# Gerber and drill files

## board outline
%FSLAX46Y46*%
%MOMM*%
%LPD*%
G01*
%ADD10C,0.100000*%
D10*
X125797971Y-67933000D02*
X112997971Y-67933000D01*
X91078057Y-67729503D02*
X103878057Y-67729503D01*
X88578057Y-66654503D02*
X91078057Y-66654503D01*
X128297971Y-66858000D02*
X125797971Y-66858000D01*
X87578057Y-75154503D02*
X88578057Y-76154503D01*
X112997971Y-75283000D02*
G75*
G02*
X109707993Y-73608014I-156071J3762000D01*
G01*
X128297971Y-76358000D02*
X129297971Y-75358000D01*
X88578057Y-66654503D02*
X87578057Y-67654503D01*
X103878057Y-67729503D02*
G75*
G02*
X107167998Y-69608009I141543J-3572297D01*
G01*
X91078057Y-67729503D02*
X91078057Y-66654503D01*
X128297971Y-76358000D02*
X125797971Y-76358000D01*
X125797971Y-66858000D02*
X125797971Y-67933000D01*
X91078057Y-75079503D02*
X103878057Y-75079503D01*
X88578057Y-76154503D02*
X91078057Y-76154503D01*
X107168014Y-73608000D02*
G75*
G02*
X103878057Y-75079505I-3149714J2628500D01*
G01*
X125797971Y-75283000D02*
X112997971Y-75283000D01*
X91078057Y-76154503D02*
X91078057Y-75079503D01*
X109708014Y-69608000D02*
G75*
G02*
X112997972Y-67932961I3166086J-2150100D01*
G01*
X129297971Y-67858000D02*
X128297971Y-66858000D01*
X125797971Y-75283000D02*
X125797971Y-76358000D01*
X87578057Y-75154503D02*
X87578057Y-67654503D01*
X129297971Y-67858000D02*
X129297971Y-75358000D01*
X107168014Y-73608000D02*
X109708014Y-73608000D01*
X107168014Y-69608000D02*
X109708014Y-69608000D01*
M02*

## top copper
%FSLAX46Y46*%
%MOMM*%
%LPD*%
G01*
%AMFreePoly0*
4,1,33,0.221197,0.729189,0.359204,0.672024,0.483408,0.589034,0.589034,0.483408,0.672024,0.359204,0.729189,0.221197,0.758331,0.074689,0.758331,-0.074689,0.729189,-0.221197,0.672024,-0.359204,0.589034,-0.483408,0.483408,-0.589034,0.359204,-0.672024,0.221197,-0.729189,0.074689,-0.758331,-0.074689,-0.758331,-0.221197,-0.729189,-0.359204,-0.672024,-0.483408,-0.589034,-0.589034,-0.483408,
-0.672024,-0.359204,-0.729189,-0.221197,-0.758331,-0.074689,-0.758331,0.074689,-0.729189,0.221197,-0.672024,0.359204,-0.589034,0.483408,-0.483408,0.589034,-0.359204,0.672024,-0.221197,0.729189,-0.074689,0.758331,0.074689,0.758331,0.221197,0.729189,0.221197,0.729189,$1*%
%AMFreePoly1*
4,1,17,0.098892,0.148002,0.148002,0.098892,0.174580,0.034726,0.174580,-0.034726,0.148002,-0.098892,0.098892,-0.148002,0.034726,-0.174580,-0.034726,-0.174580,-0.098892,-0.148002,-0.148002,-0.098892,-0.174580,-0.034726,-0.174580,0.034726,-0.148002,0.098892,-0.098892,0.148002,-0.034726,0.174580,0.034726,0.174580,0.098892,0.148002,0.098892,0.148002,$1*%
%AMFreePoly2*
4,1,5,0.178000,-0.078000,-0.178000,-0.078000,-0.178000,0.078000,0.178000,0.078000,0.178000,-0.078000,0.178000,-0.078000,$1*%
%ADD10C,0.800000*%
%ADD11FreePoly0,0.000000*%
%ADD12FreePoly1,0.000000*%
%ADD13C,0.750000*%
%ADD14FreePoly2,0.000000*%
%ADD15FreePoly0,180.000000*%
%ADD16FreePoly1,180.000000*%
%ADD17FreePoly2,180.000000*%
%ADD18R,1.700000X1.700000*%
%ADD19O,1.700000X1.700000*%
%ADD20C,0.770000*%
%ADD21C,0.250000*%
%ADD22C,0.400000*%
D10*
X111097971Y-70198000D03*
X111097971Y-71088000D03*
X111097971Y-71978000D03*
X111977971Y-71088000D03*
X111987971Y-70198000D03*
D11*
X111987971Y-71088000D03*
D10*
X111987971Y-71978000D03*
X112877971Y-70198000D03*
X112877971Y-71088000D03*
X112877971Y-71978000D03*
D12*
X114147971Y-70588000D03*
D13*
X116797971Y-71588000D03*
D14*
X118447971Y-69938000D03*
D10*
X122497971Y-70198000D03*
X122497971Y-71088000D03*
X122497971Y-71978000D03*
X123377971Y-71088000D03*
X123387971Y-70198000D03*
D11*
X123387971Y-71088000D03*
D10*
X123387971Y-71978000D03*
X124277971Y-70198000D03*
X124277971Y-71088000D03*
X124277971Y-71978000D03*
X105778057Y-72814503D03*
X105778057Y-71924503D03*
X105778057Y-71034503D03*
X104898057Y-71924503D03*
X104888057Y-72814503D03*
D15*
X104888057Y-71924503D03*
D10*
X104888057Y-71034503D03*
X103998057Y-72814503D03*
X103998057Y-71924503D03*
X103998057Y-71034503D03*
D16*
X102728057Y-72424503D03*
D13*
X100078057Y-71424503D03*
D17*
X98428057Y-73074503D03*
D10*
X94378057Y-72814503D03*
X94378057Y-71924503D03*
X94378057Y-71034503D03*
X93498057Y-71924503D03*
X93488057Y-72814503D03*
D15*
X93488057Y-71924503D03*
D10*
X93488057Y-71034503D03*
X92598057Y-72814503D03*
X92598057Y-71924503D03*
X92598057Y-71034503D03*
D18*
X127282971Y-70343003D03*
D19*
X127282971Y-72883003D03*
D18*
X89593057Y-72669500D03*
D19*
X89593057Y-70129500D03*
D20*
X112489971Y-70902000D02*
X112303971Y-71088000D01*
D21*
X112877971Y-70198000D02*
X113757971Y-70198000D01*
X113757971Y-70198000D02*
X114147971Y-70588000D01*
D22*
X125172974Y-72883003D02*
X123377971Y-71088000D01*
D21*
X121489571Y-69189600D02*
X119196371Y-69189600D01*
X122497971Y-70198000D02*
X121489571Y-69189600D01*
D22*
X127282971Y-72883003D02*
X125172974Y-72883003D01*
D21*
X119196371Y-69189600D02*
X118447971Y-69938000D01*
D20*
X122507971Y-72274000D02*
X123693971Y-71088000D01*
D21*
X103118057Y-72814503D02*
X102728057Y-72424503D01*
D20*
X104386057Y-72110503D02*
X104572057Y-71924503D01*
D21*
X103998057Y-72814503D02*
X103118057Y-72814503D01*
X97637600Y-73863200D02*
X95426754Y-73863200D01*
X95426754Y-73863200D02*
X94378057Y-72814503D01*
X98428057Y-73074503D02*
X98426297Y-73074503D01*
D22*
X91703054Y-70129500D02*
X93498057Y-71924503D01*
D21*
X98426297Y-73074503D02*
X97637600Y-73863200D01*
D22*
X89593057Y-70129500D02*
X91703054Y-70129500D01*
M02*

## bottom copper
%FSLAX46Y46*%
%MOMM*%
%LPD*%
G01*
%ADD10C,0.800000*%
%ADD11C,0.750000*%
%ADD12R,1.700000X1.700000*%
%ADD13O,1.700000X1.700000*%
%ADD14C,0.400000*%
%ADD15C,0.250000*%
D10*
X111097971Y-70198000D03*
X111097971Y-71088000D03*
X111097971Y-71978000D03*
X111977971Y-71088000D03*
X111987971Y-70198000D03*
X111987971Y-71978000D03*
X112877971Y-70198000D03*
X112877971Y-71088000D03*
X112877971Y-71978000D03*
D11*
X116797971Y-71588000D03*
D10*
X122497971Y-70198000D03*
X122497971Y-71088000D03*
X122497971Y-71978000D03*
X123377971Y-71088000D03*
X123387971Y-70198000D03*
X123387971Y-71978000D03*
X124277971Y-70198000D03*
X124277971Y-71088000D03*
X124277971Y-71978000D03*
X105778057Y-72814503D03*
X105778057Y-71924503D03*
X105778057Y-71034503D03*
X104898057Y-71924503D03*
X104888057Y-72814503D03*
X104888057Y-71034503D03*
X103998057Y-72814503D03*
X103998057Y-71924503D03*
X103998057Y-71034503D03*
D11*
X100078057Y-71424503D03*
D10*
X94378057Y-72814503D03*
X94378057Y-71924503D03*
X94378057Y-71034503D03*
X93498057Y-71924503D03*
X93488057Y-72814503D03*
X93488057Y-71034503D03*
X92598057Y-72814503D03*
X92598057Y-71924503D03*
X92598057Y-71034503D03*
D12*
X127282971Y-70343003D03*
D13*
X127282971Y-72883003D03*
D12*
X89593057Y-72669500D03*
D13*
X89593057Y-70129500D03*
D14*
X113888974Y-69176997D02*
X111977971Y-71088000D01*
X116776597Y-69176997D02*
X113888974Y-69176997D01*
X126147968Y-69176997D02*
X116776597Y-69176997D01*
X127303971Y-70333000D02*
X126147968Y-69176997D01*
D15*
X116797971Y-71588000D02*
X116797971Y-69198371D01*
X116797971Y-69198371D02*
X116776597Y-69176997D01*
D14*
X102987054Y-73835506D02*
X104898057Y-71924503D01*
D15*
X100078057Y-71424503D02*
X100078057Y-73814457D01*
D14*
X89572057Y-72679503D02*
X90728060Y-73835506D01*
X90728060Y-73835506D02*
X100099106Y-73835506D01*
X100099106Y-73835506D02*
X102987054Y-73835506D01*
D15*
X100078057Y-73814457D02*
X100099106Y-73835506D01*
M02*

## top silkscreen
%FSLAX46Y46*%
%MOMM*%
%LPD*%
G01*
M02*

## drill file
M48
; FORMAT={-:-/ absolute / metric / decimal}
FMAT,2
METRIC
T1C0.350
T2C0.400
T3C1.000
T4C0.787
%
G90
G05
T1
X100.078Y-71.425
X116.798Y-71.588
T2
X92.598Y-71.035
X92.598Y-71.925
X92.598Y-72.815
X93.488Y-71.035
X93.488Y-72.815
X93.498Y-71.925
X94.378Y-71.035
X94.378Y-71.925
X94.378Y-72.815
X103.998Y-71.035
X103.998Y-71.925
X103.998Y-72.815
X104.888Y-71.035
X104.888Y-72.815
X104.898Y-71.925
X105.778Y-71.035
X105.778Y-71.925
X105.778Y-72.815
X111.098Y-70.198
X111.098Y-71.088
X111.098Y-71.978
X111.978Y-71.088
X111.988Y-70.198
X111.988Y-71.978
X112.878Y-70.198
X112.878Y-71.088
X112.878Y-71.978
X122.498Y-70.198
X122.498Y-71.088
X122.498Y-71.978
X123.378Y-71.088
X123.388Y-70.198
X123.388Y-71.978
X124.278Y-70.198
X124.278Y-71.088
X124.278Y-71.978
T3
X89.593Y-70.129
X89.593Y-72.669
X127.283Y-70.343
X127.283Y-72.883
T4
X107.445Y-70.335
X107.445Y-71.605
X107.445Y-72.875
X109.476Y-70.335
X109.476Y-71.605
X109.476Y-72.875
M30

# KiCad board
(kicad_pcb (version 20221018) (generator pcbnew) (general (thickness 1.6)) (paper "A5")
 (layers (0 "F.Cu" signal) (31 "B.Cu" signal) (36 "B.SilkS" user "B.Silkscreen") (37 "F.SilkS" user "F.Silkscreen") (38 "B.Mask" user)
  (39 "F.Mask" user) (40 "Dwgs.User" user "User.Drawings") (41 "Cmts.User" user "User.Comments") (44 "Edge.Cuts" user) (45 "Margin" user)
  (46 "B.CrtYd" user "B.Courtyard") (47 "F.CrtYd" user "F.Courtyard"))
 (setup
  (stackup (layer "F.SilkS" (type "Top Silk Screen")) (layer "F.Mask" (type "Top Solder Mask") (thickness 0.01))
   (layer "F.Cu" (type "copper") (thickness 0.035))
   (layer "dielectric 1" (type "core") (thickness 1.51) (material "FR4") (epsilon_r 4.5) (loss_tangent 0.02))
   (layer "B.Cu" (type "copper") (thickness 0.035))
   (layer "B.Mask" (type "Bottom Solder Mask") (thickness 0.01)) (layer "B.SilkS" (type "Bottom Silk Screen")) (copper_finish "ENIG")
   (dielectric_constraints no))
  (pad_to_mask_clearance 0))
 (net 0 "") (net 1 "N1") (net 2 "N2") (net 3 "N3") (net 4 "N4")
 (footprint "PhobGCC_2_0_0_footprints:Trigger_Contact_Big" (layer "F.Cu") (at 116.797971 71.588)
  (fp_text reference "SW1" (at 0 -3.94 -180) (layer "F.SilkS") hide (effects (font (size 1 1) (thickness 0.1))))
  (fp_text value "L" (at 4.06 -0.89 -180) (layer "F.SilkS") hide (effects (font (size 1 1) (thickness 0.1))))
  (pad "1" thru_hole circle (at -5.7 -1.39) (size 0.8 0.8) (drill 0.4) (layers "*.Cu" "*.Mask") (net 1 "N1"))
  (pad "1" thru_hole circle (at -5.7 -0.5) (size 0.8 0.8) (drill 0.4) (layers "*.Cu" "*.Mask") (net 1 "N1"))
  (pad "1" thru_hole circle (at -5.7 0.39) (size 0.8 0.8) (drill 0.4) (layers "*.Cu" "*.Mask") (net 1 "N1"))
  (pad "1" thru_hole circle (at -4.82 -0.5) (size 0.8 0.8) (drill 0.4) (layers "*.Cu" "*.Mask") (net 1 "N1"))
  (pad "1" thru_hole circle (at -4.81 -1.39) (size 0.8 0.8) (drill 0.4) (layers "*.Cu" "*.Mask") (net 1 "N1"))
  (pad "1" smd custom (at -4.81 -0.5) (size 1.524 1.524) (layers "F.Cu" "F.Paste" "F.Mask") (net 1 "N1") (thermal_bridge_angle 45)
   (options (clearance outline) (anchor circle)) (primitives))
  (pad "1" thru_hole circle (at -4.81 0.39) (size 0.8 0.8) (drill 0.4) (layers "*.Cu" "*.Mask") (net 1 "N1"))
  (pad "1" thru_hole circle (at -3.92 -1.39) (size 0.8 0.8) (drill 0.4) (layers "*.Cu" "*.Mask") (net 1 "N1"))
  (pad "1" thru_hole circle (at -3.92 -0.5) (size 0.8 0.8) (drill 0.4) (layers "*.Cu" "*.Mask") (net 1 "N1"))
  (pad "1" thru_hole circle (at -3.92 0.39) (size 0.8 0.8) (drill 0.4) (layers "*.Cu" "*.Mask") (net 1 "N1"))
  (pad "1" smd custom (at -2.65 -1) (size 0.356 0.356) (layers "F.Cu" "F.Paste" "F.Mask") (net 1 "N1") (thermal_bridge_angle 45)
   (options (clearance outline) (anchor circle)) (primitives))
  (pad "1" thru_hole circle (at 0 0) (size 0.75 0.75) (drill 0.35) (layers "*.Cu" "*.Mask") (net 1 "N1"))
  (pad "2" smd custom (at 1.65 -1.65) (size 0.356 0.156) (layers "F.Cu" "F.Paste" "F.Mask") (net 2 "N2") (thermal_bridge_angle 45)
   (options (clearance outline) (anchor rect)) (primitives))
  (pad "2" thru_hole circle (at 5.7 -1.39) (size 0.8 0.8) (drill 0.4) (layers "*.Cu" "*.Mask") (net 2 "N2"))
  (pad "2" thru_hole circle (at 5.7 -0.5) (size 0.8 0.8) (drill 0.4) (layers "*.Cu" "*.Mask") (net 2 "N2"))
  (pad "2" thru_hole circle (at 5.7 0.39) (size 0.8 0.8) (drill 0.4) (layers "*.Cu" "*.Mask") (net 2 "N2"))
  (pad "2" thru_hole circle (at 6.58 -0.5) (size 0.8 0.8) (drill 0.4) (layers "*.Cu" "*.Mask") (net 2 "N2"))
  (pad "2" thru_hole circle (at 6.59 -1.39) (size 0.8 0.8) (drill 0.4) (layers "*.Cu" "*.Mask") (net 2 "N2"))
  (pad "2" smd custom (at 6.59 -0.5) (size 1.524 1.524) (layers "F.Cu" "F.Paste" "F.Mask") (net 2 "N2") (thermal_bridge_angle 45)
   (options (clearance outline) (anchor circle)) (primitives))
  (pad "2" thru_hole circle (at 6.59 0.39) (size 0.8 0.8) (drill 0.4) (layers "*.Cu" "*.Mask") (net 2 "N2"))
  (pad "2" thru_hole circle (at 7.48 -1.39) (size 0.8 0.8) (drill 0.4) (layers "*.Cu" "*.Mask") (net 2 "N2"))
  (pad "2" thru_hole circle (at 7.48 -0.5) (size 0.8 0.8) (drill 0.4) (layers "*.Cu" "*.Mask") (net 2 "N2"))
  (pad "2" thru_hole circle (at 7.48 0.39) (size 0.8 0.8) (drill 0.4) (layers "*.Cu" "*.Mask") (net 2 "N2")))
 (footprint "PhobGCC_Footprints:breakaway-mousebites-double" (layer "F.Cu") (at 109.705907 71.375 90)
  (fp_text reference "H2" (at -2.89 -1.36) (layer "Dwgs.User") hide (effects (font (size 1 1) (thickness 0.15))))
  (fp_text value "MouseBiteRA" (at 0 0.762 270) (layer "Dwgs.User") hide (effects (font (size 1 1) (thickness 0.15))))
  (fp_line (start -2.233 -2.537893) (end -2.233 0.002107) (stroke (width 0.1) (type solid)) (layer "Edge.Cuts"))
  (fp_line (start 1.767 -2.537893) (end 1.767 0.002107) (stroke (width 0.1) (type solid)) (layer "Edge.Cuts"))
  (pad "" np_thru_hole circle (at -1.5 -2.26085 270) (size 0.7874 0.7874) (drill 0.7874) (layers "*.Cu" "*.Mask"))
  (pad "" np_thru_hole circle (at -1.5 -0.23 90) (size 0.7874 0.7874) (drill 0.7874) (layers "*.Cu" "*.Mask"))
  (pad "" np_thru_hole circle (at -0.23 -2.26085 270) (size 0.7874 0.7874) (drill 0.7874) (layers "*.Cu" "*.Mask"))
  (pad "" np_thru_hole circle (at -0.23 -0.23 90) (size 0.7874 0.7874) (drill 0.7874) (layers "*.Cu" "*.Mask"))
  (pad "" np_thru_hole circle (at 1.04 -2.26085 270) (size 0.7874 0.7874) (drill 0.7874) (layers "*.Cu" "*.Mask"))
  (pad "" np_thru_hole circle (at 1.04 -0.23 90) (size 0.7874 0.7874) (drill 0.7874) (layers "*.Cu" "*.Mask")))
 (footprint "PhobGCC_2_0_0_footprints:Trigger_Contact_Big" (layer "F.Cu") (at 100.078057 71.424503 180)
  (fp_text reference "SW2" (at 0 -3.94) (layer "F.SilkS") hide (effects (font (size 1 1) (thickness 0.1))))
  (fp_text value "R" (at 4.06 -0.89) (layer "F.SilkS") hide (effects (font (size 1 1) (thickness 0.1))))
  (pad "1" thru_hole circle (at -5.7 -1.39 180) (size 0.8 0.8) (drill 0.4) (layers "*.Cu" "*.Mask") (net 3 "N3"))
  (pad "1" thru_hole circle (at -5.7 -0.5 180) (size 0.8 0.8) (drill 0.4) (layers "*.Cu" "*.Mask") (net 3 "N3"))
  (pad "1" thru_hole circle (at -5.7 0.39 180) (size 0.8 0.8) (drill 0.4) (layers "*.Cu" "*.Mask") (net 3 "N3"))
  (pad "1" thru_hole circle (at -4.82 -0.5 180) (size 0.8 0.8) (drill 0.4) (layers "*.Cu" "*.Mask") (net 3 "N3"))
  (pad "1" thru_hole circle (at -4.81 -1.39 180) (size 0.8 0.8) (drill 0.4) (layers "*.Cu" "*.Mask") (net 3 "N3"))
  (pad "1" smd custom (at -4.81 -0.5 180) (size 1.524 1.524) (layers "F.Cu" "F.Paste" "F.Mask") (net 3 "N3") (thermal_bridge_angle 45)
   (options (clearance outline) (anchor circle)) (primitives))
  (pad "1" thru_hole circle (at -4.81 0.39 180) (size 0.8 0.8) (drill 0.4) (layers "*.Cu" "*.Mask") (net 3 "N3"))
  (pad "1" thru_hole circle (at -3.92 -1.39 180) (size 0.8 0.8) (drill 0.4) (layers "*.Cu" "*.Mask") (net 3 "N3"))
  (pad "1" thru_hole circle (at -3.92 -0.5 180) (size 0.8 0.8) (drill 0.4) (layers "*.Cu" "*.Mask") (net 3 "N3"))
  (pad "1" thru_hole circle (at -3.92 0.39 180) (size 0.8 0.8) (drill 0.4) (layers "*.Cu" "*.Mask") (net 3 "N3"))
  (pad "1" smd custom (at -2.65 -1 180) (size 0.356 0.356) (layers "F.Cu" "F.Paste" "F.Mask") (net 3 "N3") (thermal_bridge_angle 45)
   (options (clearance outline) (anchor circle)) (primitives))
  (pad "1" thru_hole circle (at 0 0 180) (size 0.75 0.75) (drill 0.35) (layers "*.Cu" "*.Mask") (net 3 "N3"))
  (pad "2" smd custom (at 1.65 -1.65 180) (size 0.356 0.156) (layers "F.Cu" "F.Paste" "F.Mask") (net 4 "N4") (thermal_bridge_angle 45)
   (options (clearance outline) (anchor rect)) (primitives))
  (pad "2" thru_hole circle (at 5.7 -1.39 180) (size 0.8 0.8) (drill 0.4) (layers "*.Cu" "*.Mask") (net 4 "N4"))
  (pad "2" thru_hole circle (at 5.7 -0.5 180) (size 0.8 0.8) (drill 0.4) (layers "*.Cu" "*.Mask") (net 4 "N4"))
  (pad "2" thru_hole circle (at 5.7 0.39 180) (size 0.8 0.8) (drill 0.4) (layers "*.Cu" "*.Mask") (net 4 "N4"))
  (pad "2" thru_hole circle (at 6.58 -0.5 180) (size 0.8 0.8) (drill 0.4) (layers "*.Cu" "*.Mask") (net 4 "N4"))
  (pad "2" thru_hole circle (at 6.59 -1.39 180) (size 0.8 0.8) (drill 0.4) (layers "*.Cu" "*.Mask") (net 4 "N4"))
  (pad "2" smd custom (at 6.59 -0.5 180) (size 1.524 1.524) (layers "F.Cu" "F.Paste" "F.Mask") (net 4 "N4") (thermal_bridge_angle 45)
   (options (clearance outline) (anchor circle)) (primitives))
  (pad "2" thru_hole circle (at 6.59 0.39 180) (size 0.8 0.8) (drill 0.4) (layers "*.Cu" "*.Mask") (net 4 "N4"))
  (pad "2" thru_hole circle (at 7.48 -1.39 180) (size 0.8 0.8) (drill 0.4) (layers "*.Cu" "*.Mask") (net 4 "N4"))
  (pad "2" thru_hole circle (at 7.48 -0.5 180) (size 0.8 0.8) (drill 0.4) (layers "*.Cu" "*.Mask") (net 4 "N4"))
  (pad "2" thru_hole circle (at 7.48 0.39 180) (size 0.8 0.8) (drill 0.4) (layers "*.Cu" "*.Mask") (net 4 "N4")))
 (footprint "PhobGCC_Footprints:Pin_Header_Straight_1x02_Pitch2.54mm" (layer "B.Cu") (at 127.282971 70.343003 180)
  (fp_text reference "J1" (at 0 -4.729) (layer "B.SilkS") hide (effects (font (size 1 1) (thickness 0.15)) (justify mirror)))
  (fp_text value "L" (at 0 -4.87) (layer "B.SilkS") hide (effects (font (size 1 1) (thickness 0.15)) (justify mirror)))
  (pad "1" thru_hole rect (at 0 0 180) (size 1.7 1.7) (drill 1) (layers "*.Cu" "*.Mask") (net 1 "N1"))
  (pad "2" thru_hole oval (at 0 -2.54 180) (size 1.7 1.7) (drill 1) (layers "*.Cu" "*.Mask") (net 2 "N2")))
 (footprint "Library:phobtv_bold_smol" (layer "B.Cu") (at 118.4 71.7)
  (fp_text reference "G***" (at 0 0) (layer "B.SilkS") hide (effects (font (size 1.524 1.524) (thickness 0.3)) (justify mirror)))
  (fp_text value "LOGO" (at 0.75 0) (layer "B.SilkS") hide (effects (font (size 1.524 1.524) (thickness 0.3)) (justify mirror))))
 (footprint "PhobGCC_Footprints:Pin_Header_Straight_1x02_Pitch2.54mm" (layer "B.Cu") (at 89.593057 72.6695)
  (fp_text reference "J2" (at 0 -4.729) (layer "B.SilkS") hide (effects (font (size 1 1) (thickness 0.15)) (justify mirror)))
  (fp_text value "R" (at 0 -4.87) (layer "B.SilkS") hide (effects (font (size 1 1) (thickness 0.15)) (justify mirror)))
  (pad "1" thru_hole rect (at 0 0) (size 1.7 1.7) (drill 1) (layers "*.Cu" "*.Mask") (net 3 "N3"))
  (pad "2" thru_hole oval (at 0 -2.54) (size 1.7 1.7) (drill 1) (layers "*.Cu" "*.Mask") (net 4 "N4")))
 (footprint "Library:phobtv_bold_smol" (layer "B.Cu") (at 98.5 71.3 180)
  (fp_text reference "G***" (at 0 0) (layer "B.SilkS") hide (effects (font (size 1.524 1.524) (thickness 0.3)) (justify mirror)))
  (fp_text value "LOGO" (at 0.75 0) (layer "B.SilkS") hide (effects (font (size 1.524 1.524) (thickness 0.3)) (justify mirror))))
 (gr_line (start 125.797971 67.933) (end 112.997971 67.933) (stroke (width 0.1) (type solid)) (layer "Edge.Cuts"))
 (gr_line (start 91.078057 67.729503) (end 103.878057 67.729503) (stroke (width 0.1) (type solid)) (layer "Edge.Cuts"))
 (gr_line (start 88.578057 66.654503) (end 91.078057 66.654503) (stroke (width 0.1) (type solid)) (layer "Edge.Cuts"))
 (gr_line (start 128.297971 66.858) (end 125.797971 66.858) (stroke (width 0.1) (type solid)) (layer "Edge.Cuts"))
 (gr_line (start 87.578057 75.154503) (end 88.578057 76.154503) (stroke (width 0.1) (type solid)) (layer "Edge.Cuts"))
 (gr_arc (start 112.997971 75.283) (mid 111.133614 74.876392) (end 109.708014 73.608) (stroke (width 0.1) (type solid)) (layer "Edge.Cuts"))
 (gr_line (start 128.297971 76.358) (end 129.297971 75.358) (stroke (width 0.1) (type solid)) (layer "Edge.Cuts"))
 (gr_line (start 88.578057 66.654503) (end 87.578057 67.654503) (stroke (width 0.1) (type solid)) (layer "Edge.Cuts"))
 (gr_arc (start 103.878057 67.729503) (mid 105.792312 68.197147) (end 107.168014 69.608) (stroke (width 0.1) (type solid))
  (layer "Edge.Cuts"))
 (gr_line (start 91.078057 67.729503) (end 91.078057 66.654503) (stroke (width 0.1) (type solid)) (layer "Edge.Cuts"))
 (gr_line (start 128.297971 76.358) (end 125.797971 76.358) (stroke (width 0.1) (type solid)) (layer "Edge.Cuts"))
 (gr_line (start 125.797971 66.858) (end 125.797971 67.933) (stroke (width 0.1) (type solid)) (layer "Edge.Cuts"))
 (gr_line (start 91.078057 75.079503) (end 103.878057 75.079503) (stroke (width 0.1) (type solid)) (layer "Edge.Cuts"))
 (gr_line (start 88.578057 76.154503) (end 91.078057 76.154503) (stroke (width 0.1) (type solid)) (layer "Edge.Cuts"))
 (gr_arc (start 107.168014 73.608) (mid 105.69328 74.724381) (end 103.878057 75.079503) (stroke (width 0.1) (type solid))
  (layer "Edge.Cuts"))
 (gr_line (start 125.797971 75.283) (end 112.997971 75.283) (stroke (width 0.1) (type solid)) (layer "Edge.Cuts"))
 (gr_line (start 91.078057 76.154503) (end 91.078057 75.079503) (stroke (width 0.1) (type solid)) (layer "Edge.Cuts"))
 (gr_arc (start 109.708014 69.608) (mid 111.137673 68.347575) (end 112.997971 67.933) (stroke (width 0.1) (type solid)) (layer "Edge.Cuts"))
 (gr_line (start 129.297971 67.858) (end 128.297971 66.858) (stroke (width 0.1) (type solid)) (layer "Edge.Cuts"))
 (gr_line (start 125.797971 75.283) (end 125.797971 76.358) (stroke (width 0.1) (type solid)) (layer "Edge.Cuts"))
 (gr_line (start 87.578057 75.154503) (end 87.578057 67.654503) (stroke (width 0.1) (type solid)) (layer "Edge.Cuts"))
 (gr_line (start 129.297971 67.858) (end 129.297971 75.358) (stroke (width 0.1) (type solid)) (layer "Edge.Cuts"))
 (segment (start 112.489971 70.902) (end 112.303971 71.088) (width 0.77) (layer "F.Cu") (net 1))
 (segment (start 112.877971 70.198) (end 113.757971 70.198) (width 0.25) (layer "F.Cu") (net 1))
 (segment (start 113.757971 70.198) (end 114.147971 70.588) (width 0.25) (layer "F.Cu") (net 1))
 (segment (start 113.888974 69.176997) (end 111.977971 71.088) (width 0.4) (layer "B.Cu") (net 1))
 (segment (start 116.776597 69.176997) (end 113.888974 69.176997) (width 0.4) (layer "B.Cu") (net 1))
 (segment (start 126.147968 69.176997) (end 116.776597 69.176997) (width 0.4) (layer "B.Cu") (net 1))
 (segment (start 127.303971 70.333) (end 126.147968 69.176997) (width 0.4) (layer "B.Cu") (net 1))
 (segment (start 116.797971 71.588) (end 116.797971 69.198371) (width 0.25) (layer "B.Cu") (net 1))
 (segment (start 116.797971 69.198371) (end 116.776597 69.176997) (width 0.25) (layer "B.Cu") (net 1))
 (segment (start 125.172974 72.883003) (end 123.377971 71.088) (width 0.4) (layer "F.Cu") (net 2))
 (segment (start 121.489571 69.1896) (end 119.196371 69.1896) (width 0.25) (layer "F.Cu") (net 2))
 (segment (start 122.497971 70.198) (end 121.489571 69.1896) (width 0.25) (layer "F.Cu") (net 2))
 (segment (start 127.282971 72.883003) (end 125.172974 72.883003) (width 0.4) (layer "F.Cu") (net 2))
 (segment (start 119.196371 69.1896) (end 118.447971 69.938) (width 0.25) (layer "F.Cu") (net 2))
 (segment (start 122.507971 72.274) (end 123.693971 71.088) (width 0.77) (layer "F.Cu") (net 2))
 (segment (start 103.118057 72.814503) (end 102.728057 72.424503) (width 0.25) (layer "F.Cu") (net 3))
 (segment (start 104.386057 72.110503) (end 104.572057 71.924503) (width 0.77) (layer "F.Cu") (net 3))
 (segment (start 103.998057 72.814503) (end 103.118057 72.814503) (width 0.25) (layer "F.Cu") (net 3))
 (segment (start 102.987054 73.835506) (end 104.898057 71.924503) (width 0.4) (layer "B.Cu") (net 3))
 (segment (start 100.078057 71.424503) (end 100.078057 73.814457) (width 0.25) (layer "B.Cu") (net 3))
 (segment (start 89.572057 72.679503) (end 90.72806 73.835506) (width 0.4) (layer "B.Cu") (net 3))
 (segment (start 90.72806 73.835506) (end 100.099106 73.835506) (width 0.4) (layer "B.Cu") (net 3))
 (segment (start 100.099106 73.835506) (end 102.987054 73.835506) (width 0.4) (layer "B.Cu") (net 3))
 (segment (start 100.078057 73.814457) (end 100.099106 73.835506) (width 0.25) (layer "B.Cu") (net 3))
 (segment (start 97.6376 73.8632) (end 95.426754 73.8632) (width 0.25) (layer "F.Cu") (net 4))
 (segment (start 95.426754 73.8632) (end 94.378057 72.814503) (width 0.25) (layer "F.Cu") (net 4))
 (segment (start 98.428057 73.074503) (end 98.426297 73.074503) (width 0.25) (layer "F.Cu") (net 4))
 (segment (start 91.703054 70.1295) (end 93.498057 71.924503) (width 0.4) (layer "F.Cu") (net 4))
 (segment (start 98.426297 73.074503) (end 97.6376 73.8632) (width 0.25) (layer "F.Cu") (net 4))
 (segment (start 89.593057 70.1295) (end 91.703054 70.1295) (width 0.4) (layer "F.Cu") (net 4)))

